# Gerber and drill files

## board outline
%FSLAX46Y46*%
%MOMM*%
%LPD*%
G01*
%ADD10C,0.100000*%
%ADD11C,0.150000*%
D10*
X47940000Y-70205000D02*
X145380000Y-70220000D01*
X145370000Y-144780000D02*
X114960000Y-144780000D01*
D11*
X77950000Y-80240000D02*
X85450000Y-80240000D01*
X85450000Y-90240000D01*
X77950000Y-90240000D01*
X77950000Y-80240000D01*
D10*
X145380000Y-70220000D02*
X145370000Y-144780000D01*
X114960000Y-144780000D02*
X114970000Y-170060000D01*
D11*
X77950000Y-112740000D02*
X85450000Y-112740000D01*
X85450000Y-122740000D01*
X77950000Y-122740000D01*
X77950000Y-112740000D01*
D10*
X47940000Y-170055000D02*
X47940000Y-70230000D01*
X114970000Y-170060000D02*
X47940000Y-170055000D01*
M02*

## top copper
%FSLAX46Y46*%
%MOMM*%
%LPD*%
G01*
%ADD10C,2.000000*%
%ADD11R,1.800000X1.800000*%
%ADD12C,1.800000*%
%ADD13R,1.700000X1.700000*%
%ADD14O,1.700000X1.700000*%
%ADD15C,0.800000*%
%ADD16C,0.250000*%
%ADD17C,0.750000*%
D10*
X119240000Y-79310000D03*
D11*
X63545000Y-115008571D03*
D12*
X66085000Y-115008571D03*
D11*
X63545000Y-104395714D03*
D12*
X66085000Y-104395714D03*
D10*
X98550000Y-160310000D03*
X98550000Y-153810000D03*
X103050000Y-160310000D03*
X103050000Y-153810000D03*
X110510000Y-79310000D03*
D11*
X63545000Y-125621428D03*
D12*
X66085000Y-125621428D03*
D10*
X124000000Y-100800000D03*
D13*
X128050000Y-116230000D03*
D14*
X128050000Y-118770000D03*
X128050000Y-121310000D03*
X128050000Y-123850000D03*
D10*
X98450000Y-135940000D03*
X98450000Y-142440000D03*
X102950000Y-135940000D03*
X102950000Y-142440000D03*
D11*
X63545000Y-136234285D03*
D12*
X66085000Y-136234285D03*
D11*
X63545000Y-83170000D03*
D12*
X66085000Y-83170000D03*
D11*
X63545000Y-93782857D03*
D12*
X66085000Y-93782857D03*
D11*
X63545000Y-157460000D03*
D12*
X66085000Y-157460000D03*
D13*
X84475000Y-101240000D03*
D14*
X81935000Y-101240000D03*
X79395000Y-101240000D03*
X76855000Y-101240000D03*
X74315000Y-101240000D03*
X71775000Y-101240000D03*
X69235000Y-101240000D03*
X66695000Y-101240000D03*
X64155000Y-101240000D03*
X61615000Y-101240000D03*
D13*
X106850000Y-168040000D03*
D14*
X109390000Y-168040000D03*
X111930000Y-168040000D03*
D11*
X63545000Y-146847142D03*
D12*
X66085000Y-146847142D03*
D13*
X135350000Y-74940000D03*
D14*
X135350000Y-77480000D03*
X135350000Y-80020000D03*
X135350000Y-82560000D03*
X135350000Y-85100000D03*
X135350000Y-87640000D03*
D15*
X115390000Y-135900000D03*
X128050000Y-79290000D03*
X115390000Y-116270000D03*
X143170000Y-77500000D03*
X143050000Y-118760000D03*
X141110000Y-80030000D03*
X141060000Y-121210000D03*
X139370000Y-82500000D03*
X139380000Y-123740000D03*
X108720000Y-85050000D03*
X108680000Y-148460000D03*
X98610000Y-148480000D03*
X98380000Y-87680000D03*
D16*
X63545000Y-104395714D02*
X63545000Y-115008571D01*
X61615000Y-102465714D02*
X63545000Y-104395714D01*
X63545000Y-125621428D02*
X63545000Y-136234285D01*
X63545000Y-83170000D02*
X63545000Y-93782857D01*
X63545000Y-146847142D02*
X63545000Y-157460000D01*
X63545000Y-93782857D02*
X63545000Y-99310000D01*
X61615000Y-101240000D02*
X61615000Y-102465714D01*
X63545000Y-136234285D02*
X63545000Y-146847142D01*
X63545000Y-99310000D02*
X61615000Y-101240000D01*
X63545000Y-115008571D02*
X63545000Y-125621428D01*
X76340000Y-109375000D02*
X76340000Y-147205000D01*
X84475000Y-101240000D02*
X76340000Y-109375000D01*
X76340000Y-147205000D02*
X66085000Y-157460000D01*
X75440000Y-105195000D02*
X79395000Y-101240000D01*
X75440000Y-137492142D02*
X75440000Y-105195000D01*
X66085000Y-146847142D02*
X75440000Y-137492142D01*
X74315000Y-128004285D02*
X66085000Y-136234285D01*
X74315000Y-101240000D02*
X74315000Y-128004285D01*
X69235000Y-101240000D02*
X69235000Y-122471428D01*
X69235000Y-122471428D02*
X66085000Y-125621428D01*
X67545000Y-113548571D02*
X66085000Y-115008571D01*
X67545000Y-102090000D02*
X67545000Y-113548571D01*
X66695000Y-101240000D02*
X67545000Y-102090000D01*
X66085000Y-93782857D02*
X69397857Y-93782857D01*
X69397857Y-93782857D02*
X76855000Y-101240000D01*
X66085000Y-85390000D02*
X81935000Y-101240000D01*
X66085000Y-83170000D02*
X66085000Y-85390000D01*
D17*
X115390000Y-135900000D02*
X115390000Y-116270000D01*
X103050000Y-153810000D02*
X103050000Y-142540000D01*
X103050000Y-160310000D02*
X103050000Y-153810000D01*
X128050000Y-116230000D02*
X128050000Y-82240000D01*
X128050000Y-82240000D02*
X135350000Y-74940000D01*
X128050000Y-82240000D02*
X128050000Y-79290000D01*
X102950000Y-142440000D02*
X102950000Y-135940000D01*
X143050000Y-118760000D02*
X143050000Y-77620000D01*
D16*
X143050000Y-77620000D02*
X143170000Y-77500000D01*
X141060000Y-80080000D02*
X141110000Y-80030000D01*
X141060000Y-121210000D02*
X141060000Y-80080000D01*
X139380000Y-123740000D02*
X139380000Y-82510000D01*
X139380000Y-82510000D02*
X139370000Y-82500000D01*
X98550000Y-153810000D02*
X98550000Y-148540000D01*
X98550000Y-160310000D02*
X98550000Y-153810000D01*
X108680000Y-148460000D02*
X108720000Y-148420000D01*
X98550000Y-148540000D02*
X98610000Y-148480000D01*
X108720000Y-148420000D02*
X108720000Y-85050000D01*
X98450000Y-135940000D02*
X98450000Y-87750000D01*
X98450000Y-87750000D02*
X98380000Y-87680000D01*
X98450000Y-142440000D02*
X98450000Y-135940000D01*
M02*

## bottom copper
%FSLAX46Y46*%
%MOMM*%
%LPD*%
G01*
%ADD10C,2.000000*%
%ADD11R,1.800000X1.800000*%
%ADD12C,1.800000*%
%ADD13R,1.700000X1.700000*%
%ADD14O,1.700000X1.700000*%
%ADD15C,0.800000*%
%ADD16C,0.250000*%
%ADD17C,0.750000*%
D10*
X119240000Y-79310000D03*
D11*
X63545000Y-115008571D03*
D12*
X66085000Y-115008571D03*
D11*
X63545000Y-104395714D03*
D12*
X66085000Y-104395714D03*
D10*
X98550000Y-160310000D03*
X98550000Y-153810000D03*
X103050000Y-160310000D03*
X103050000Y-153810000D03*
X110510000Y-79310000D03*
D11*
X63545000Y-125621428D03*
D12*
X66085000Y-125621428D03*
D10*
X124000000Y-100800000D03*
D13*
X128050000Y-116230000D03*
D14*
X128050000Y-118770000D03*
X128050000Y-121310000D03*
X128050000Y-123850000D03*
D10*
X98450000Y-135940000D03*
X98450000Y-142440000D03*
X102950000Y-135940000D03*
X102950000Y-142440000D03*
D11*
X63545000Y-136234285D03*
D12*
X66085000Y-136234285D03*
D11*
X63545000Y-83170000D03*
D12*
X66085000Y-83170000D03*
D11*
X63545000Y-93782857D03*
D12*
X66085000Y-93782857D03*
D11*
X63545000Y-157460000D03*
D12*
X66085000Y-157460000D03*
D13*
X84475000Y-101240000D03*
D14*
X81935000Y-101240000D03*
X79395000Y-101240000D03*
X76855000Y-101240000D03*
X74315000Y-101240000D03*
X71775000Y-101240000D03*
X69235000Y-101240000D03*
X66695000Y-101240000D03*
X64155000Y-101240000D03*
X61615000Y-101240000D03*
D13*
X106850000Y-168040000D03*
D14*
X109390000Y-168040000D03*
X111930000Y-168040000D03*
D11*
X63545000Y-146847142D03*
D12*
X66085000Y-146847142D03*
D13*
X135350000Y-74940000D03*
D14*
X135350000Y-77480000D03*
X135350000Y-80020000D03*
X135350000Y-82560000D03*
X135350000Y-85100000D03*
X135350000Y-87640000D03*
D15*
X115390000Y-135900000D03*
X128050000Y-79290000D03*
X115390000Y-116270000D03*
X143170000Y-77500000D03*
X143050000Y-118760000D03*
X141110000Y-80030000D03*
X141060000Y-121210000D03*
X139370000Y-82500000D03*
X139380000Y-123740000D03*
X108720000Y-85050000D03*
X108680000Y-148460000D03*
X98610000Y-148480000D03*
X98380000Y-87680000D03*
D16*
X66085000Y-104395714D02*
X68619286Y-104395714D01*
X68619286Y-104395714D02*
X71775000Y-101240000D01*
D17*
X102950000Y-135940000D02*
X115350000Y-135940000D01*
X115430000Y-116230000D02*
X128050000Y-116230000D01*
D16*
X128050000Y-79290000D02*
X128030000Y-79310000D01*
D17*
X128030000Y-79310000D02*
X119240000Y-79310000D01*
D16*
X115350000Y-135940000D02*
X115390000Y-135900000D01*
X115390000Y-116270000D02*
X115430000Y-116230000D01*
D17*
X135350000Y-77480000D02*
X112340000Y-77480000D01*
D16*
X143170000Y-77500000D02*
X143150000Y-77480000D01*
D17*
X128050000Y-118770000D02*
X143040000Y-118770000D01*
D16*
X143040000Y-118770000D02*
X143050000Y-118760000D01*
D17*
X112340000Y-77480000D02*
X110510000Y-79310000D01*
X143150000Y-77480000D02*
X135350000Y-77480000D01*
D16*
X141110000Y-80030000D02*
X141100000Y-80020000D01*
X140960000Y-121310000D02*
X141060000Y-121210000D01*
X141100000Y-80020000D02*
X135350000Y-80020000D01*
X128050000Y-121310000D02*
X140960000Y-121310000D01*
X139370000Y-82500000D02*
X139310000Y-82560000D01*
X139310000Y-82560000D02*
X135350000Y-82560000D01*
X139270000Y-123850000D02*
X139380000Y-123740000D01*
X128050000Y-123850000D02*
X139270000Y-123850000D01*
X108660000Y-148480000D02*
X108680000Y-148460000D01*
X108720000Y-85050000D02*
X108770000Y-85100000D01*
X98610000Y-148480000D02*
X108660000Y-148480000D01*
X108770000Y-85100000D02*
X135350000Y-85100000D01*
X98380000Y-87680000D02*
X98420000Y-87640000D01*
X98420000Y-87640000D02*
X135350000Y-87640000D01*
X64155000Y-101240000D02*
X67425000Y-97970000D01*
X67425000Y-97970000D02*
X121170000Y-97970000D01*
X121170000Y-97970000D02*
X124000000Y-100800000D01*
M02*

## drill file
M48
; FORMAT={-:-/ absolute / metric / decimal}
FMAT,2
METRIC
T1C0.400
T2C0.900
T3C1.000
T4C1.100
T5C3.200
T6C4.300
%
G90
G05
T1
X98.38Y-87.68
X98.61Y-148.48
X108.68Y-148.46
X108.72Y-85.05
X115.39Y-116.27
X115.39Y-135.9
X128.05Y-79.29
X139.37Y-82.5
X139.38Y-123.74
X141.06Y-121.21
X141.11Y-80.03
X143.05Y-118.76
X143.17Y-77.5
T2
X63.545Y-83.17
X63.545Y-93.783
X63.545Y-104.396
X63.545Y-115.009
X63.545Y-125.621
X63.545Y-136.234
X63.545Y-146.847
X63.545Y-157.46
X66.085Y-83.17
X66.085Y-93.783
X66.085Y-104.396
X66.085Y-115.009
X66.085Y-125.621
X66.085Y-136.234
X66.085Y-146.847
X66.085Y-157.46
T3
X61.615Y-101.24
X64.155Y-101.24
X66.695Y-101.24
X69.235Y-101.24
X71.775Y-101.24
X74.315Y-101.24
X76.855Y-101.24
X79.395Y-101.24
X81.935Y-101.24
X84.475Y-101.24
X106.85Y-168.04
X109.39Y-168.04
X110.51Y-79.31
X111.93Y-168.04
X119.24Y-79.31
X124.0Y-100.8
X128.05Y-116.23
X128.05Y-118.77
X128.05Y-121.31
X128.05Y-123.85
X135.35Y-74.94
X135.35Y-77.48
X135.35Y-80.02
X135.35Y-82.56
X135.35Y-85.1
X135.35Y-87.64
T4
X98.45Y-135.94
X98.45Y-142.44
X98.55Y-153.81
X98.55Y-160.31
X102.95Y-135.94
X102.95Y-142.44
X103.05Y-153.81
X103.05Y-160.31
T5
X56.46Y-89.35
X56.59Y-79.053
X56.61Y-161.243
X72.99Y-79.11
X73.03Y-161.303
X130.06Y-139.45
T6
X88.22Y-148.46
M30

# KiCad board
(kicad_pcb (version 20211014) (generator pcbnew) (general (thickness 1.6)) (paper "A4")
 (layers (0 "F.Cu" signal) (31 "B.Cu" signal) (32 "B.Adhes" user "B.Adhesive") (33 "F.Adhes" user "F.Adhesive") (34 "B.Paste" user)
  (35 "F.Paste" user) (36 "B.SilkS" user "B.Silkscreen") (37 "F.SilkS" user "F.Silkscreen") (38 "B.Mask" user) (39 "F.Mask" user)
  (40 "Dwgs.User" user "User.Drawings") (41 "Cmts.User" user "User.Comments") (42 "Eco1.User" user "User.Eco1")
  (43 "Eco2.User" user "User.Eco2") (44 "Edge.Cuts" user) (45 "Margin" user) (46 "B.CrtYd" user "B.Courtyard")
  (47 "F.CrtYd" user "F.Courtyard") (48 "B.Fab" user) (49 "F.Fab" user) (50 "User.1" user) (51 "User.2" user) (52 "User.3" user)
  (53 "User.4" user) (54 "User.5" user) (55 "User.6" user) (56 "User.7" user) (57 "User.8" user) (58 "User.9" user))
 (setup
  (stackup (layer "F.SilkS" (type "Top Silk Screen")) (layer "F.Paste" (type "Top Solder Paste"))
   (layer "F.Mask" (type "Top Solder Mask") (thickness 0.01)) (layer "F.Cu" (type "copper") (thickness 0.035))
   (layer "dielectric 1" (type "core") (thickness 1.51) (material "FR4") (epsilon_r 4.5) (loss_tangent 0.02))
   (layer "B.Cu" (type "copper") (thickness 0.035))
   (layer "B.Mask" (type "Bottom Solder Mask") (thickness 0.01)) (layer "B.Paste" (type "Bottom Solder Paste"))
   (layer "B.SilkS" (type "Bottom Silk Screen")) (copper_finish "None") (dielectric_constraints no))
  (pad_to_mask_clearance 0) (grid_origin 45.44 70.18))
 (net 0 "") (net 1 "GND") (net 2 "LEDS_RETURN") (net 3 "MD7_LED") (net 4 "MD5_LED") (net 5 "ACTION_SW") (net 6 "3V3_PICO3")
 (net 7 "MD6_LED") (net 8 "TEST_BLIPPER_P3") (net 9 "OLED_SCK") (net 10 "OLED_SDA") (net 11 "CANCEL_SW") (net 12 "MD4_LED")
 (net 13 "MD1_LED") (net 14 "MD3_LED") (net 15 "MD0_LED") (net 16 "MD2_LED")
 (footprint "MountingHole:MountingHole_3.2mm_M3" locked (layer "F.Cu") (at 130.06 139.450113)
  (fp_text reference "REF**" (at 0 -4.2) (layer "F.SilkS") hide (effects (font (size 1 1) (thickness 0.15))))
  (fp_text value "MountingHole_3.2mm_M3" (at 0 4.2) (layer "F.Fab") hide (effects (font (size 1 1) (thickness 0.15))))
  (pad "" np_thru_hole circle locked (at 0 0) (size 3.2 3.2) (drill 3.2) (layers *.Cu *.Mask)))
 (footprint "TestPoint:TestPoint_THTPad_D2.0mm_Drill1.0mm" (layer "F.Cu") (at 119.24 79.31)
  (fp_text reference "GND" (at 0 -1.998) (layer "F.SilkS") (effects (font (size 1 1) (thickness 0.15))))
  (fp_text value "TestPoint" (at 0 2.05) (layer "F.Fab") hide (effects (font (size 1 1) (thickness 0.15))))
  (pad "1" thru_hole circle (at 0 0) (size 2 2) (drill 1) (layers *.Cu *.Mask) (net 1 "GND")))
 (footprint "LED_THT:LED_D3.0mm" (layer "F.Cu") (at 63.545 115.008571)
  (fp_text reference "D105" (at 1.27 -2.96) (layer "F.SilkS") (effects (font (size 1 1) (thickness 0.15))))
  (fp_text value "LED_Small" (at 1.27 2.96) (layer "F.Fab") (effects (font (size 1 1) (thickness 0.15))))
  (pad "1" thru_hole rect (at 0 0) (size 1.8 1.8) (drill 0.9) (layers *.Cu *.Mask) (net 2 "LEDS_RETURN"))
  (pad "2" thru_hole circle (at 2.54 0) (size 1.8 1.8) (drill 0.9) (layers *.Cu *.Mask) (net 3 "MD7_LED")))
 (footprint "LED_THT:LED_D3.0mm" (layer "F.Cu") (at 63.545 104.395714)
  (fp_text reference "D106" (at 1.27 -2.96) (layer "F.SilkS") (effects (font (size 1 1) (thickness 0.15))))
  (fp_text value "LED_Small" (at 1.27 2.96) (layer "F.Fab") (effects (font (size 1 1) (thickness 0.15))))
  (pad "1" thru_hole rect (at 0 0) (size 1.8 1.8) (drill 0.9) (layers *.Cu *.Mask) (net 2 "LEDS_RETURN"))
  (pad "2" thru_hole circle (at 2.54 0) (size 1.8 1.8) (drill 0.9) (layers *.Cu *.Mask) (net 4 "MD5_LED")))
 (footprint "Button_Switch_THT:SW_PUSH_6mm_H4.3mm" (layer "F.Cu") (at 98.55 160.31 90)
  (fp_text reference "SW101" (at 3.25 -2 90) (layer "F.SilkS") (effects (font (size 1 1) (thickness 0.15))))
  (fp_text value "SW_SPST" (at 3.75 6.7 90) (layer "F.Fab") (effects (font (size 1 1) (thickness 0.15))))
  (pad "1" thru_hole circle (at 0 0 180) (size 2 2) (drill 1.1) (layers *.Cu *.Mask) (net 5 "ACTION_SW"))
  (pad "1" thru_hole circle (at 6.5 0 180) (size 2 2) (drill 1.1) (layers *.Cu *.Mask) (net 5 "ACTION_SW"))
  (pad "2" thru_hole circle (at 0 4.5 180) (size 2 2) (drill 1.1) (layers *.Cu *.Mask) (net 1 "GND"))
  (pad "2" thru_hole circle (at 6.5 4.5 180) (size 2 2) (drill 1.1) (layers *.Cu *.Mask) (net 1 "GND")))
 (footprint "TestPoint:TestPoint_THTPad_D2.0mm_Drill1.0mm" (layer "F.Cu") (at 110.51 79.31)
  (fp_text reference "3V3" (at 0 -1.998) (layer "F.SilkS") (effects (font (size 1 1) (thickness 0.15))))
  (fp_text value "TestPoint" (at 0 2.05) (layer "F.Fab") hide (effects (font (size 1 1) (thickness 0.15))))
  (pad "1" thru_hole circle (at 0 0) (size 2 2) (drill 1) (layers *.Cu *.Mask) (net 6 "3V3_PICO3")))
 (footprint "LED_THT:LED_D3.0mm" (layer "F.Cu") (at 63.545 125.621428)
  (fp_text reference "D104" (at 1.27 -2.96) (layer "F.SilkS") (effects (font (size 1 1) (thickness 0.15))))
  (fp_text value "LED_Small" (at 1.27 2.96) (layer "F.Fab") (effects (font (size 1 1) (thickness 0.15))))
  (pad "1" thru_hole rect (at 0 0) (size 1.8 1.8) (drill 0.9) (layers *.Cu *.Mask) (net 2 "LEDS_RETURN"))
  (pad "2" thru_hole circle (at 2.54 0) (size 1.8 1.8) (drill 0.9) (layers *.Cu *.Mask) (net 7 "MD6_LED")))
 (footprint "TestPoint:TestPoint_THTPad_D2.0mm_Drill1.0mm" (layer "F.Cu") (at 124 100.8)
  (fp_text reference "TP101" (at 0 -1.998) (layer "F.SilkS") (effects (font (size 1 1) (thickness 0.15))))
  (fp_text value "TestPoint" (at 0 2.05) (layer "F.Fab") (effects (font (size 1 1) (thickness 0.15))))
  (pad "1" thru_hole circle (at 0 0) (size 2 2) (drill 1) (layers *.Cu *.Mask) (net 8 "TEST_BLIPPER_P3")))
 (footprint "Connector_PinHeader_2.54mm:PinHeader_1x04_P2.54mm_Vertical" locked (layer "F.Cu") (at 128.05 116.23)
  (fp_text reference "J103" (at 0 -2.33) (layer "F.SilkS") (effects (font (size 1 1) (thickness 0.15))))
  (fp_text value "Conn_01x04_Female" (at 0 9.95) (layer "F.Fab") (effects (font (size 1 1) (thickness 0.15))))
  (pad "1" thru_hole rect locked (at 0 0) (size 1.7 1.7) (drill 1) (layers *.Cu *.Mask) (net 1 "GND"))
  (pad "2" thru_hole oval locked (at 0 2.54) (size 1.7 1.7) (drill 1) (layers *.Cu *.Mask) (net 6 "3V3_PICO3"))
  (pad "3" thru_hole oval locked (at 0 5.08) (size 1.7 1.7) (drill 1) (layers *.Cu *.Mask) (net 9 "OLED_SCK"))
  (pad "4" thru_hole oval locked (at 0 7.62) (size 1.7 1.7) (drill 1) (layers *.Cu *.Mask) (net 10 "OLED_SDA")))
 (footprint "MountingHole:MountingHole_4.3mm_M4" (layer "F.Cu") (at 88.22 148.46)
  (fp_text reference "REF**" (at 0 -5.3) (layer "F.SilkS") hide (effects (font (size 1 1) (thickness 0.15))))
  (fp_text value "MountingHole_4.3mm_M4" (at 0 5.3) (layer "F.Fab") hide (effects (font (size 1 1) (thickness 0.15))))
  (pad "" np_thru_hole circle (at 0 0) (size 4.3 4.3) (drill 4.3) (layers F&B.Cu *.Mask)))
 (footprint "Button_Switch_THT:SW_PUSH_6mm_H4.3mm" (layer "F.Cu") (at 98.45 142.44 90)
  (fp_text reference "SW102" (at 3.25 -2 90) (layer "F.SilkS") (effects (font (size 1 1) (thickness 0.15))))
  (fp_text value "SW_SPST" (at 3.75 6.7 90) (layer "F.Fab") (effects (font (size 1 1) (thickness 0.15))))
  (pad "1" thru_hole circle (at 6.5 0 180) (size 2 2) (drill 1.1) (layers *.Cu *.Mask) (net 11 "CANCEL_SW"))
  (pad "1" thru_hole circle (at 0 0 180) (size 2 2) (drill 1.1) (layers *.Cu *.Mask) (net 11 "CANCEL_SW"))
  (pad "2" thru_hole circle (at 6.5 4.5 180) (size 2 2) (drill 1.1) (layers *.Cu *.Mask) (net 1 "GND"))
  (pad "2" thru_hole circle (at 0 4.5 180) (size 2 2) (drill 1.1) (layers *.Cu *.Mask) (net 1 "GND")))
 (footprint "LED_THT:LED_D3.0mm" (layer "F.Cu") (at 63.545 136.234285)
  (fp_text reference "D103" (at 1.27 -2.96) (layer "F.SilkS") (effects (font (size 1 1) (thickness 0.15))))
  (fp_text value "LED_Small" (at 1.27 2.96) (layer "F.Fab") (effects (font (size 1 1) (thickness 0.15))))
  (pad "1" thru_hole rect (at 0 0) (size 1.8 1.8) (drill 0.9) (layers *.Cu *.Mask) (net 2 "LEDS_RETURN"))
  (pad "2" thru_hole circle (at 2.54 0) (size 1.8 1.8) (drill 0.9) (layers *.Cu *.Mask) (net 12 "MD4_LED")))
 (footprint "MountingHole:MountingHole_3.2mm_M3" (layer "F.Cu") (at 56.59 79.052856 -90)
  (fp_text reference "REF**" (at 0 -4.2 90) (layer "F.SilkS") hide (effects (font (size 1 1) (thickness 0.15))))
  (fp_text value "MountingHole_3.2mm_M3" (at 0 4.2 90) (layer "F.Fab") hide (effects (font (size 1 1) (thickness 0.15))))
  (pad "" np_thru_hole circle locked (at 0 0 270) (size 3.2 3.2) (drill 3.2) (layers F&B.Cu *.Mask)))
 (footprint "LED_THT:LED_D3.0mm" (layer "F.Cu") (at 63.545 83.17)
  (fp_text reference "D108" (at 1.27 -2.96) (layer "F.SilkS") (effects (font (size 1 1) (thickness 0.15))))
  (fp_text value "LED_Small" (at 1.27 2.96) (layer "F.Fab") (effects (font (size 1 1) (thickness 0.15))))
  (pad "1" thru_hole rect (at 0 0) (size 1.8 1.8) (drill 0.9) (layers *.Cu *.Mask) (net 2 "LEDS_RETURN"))
  (pad "2" thru_hole circle (at 2.54 0) (size 1.8 1.8) (drill 0.9) (layers *.Cu *.Mask) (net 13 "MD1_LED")))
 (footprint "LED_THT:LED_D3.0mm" (layer "F.Cu") (at 63.545 93.782857)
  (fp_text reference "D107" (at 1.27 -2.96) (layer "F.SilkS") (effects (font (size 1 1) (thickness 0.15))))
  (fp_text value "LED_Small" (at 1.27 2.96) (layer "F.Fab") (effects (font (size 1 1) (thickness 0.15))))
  (pad "1" thru_hole rect (at 0 0) (size 1.8 1.8) (drill 0.9) (layers *.Cu *.Mask) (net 2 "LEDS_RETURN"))
  (pad "2" thru_hole circle (at 2.54 0) (size 1.8 1.8) (drill 0.9) (layers *.Cu *.Mask) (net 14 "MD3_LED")))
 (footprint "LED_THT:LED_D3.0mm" (layer "F.Cu") (at 63.545 157.46)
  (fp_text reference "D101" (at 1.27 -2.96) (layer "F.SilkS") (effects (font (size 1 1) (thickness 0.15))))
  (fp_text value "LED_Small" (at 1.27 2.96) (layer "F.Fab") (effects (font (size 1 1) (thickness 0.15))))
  (pad "1" thru_hole rect (at 0 0) (size 1.8 1.8) (drill 0.9) (layers *.Cu *.Mask) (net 2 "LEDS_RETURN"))
  (pad "2" thru_hole circle (at 2.54 0) (size 1.8 1.8) (drill 0.9) (layers *.Cu *.Mask) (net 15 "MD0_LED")))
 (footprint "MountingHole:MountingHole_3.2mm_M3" (layer "F.Cu") (at 56.61 161.242856 -90)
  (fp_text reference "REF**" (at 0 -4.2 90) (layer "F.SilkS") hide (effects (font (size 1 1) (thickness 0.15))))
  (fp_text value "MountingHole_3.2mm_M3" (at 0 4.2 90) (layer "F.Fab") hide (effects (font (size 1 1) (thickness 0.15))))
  (pad "" np_thru_hole circle locked (at 0 0 270) (size 3.2 3.2) (drill 3.2) (layers F&B.Cu *.Mask)))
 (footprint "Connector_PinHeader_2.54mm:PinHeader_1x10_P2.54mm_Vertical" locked (layer "F.Cu") (at 84.475 101.24 -90)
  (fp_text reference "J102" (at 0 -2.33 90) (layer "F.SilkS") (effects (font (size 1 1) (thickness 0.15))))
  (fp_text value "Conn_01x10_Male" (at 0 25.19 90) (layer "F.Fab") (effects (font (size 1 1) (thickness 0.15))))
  (pad "1" thru_hole rect locked (at 0 0 270) (size 1.7 1.7) (drill 1) (layers *.Cu *.Mask) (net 15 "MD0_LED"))
  (pad "2" thru_hole oval locked (at 0 2.54 270) (size 1.7 1.7) (drill 1) (layers *.Cu *.Mask) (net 13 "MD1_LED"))
  (pad "3" thru_hole oval locked (at 0 5.08 270) (size 1.7 1.7) (drill 1) (layers *.Cu *.Mask) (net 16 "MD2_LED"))
  (pad "4" thru_hole oval locked (at 0 7.62 270) (size 1.7 1.7) (drill 1) (layers *.Cu *.Mask) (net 14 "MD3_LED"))
  (pad "5" thru_hole oval locked (at 0 10.16 270) (size 1.7 1.7) (drill 1) (layers *.Cu *.Mask) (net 12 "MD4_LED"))
  (pad "6" thru_hole oval locked (at 0 12.7 270) (size 1.7 1.7) (drill 1) (layers *.Cu *.Mask) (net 4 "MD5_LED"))
  (pad "7" thru_hole oval locked (at 0 15.24 270) (size 1.7 1.7) (drill 1) (layers *.Cu *.Mask) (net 7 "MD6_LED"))
  (pad "8" thru_hole oval locked (at 0 17.78 270) (size 1.7 1.7) (drill 1) (layers *.Cu *.Mask) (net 3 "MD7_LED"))
  (pad "9" thru_hole oval locked (at 0 20.32 270) (size 1.7 1.7) (drill 1) (layers *.Cu *.Mask) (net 8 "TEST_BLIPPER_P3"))
  (pad "10" thru_hole oval locked (at 0 22.86 270) (size 1.7 1.7) (drill 1) (layers *.Cu *.Mask) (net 2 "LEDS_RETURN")))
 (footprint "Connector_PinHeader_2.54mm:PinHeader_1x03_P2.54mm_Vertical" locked (layer "F.Cu") (at 106.85 168.04 90)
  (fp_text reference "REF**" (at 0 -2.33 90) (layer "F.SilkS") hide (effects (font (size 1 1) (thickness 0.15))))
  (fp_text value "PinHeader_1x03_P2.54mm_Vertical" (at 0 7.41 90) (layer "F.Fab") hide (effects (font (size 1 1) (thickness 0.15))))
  (pad "1" thru_hole rect locked (at 0 0 90) (size 1.7 1.7) (drill 1) (layers F&B.Cu *.Mask))
  (pad "2" thru_hole oval locked (at 0 2.54 90) (size 1.7 1.7) (drill 1) (layers F&B.Cu *.Mask))
  (pad "3" thru_hole oval locked (at 0 5.08 90) (size 1.7 1.7) (drill 1) (layers F&B.Cu *.Mask)))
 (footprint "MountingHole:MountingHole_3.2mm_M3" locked (layer "F.Cu") (at 56.46 89.350113)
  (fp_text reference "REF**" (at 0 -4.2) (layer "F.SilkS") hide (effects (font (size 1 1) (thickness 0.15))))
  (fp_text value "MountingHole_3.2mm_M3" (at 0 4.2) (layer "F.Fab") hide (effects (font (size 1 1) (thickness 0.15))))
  (pad "" np_thru_hole circle locked (at 0 0) (size 3.2 3.2) (drill 3.2) (layers *.Cu *.Mask)))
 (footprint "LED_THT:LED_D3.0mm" (layer "F.Cu") (at 63.545 146.847142)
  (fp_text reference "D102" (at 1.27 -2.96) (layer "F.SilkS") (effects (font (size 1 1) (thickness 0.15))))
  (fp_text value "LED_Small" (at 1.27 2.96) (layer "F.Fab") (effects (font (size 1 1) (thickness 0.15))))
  (pad "1" thru_hole rect (at 0 0) (size 1.8 1.8) (drill 0.9) (layers *.Cu *.Mask) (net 2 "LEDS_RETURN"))
  (pad "2" thru_hole circle (at 2.54 0) (size 1.8 1.8) (drill 0.9) (layers *.Cu *.Mask) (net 16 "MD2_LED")))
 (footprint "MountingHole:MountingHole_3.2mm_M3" (layer "F.Cu") (at 73.03 161.302856 -90)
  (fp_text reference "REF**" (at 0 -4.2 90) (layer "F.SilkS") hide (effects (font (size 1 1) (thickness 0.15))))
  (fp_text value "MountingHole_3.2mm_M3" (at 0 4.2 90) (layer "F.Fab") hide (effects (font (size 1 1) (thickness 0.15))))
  (pad "" np_thru_hole circle locked (at 0 0 270) (size 3.2 3.2) (drill 3.2) (layers F&B.Cu *.Mask)))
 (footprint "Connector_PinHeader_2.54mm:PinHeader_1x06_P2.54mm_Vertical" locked (layer "F.Cu") (at 135.35 74.94)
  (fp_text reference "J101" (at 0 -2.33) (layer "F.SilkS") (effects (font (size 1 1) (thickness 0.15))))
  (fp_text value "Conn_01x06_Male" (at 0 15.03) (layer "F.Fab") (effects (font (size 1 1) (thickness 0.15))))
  (pad "1" thru_hole rect locked (at 0 0) (size 1.7 1.7) (drill 1) (layers *.Cu *.Mask) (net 1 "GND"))
  (pad "2" thru_hole oval locked (at 0 2.54) (size 1.7 1.7) (drill 1) (layers *.Cu *.Mask) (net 6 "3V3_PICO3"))
  (pad "3" thru_hole oval locked (at 0 5.08) (size 1.7 1.7) (drill 1) (layers *.Cu *.Mask) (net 9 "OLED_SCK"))
  (pad "4" thru_hole oval locked (at 0 7.62) (size 1.7 1.7) (drill 1) (layers *.Cu *.Mask) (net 10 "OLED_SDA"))
  (pad "5" thru_hole oval locked (at 0 10.16) (size 1.7 1.7) (drill 1) (layers *.Cu *.Mask) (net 5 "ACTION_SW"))
  (pad "6" thru_hole oval locked (at 0 12.7) (size 1.7 1.7) (drill 1) (layers *.Cu *.Mask) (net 11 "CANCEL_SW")))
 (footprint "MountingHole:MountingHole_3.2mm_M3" (layer "F.Cu") (at 72.99 79.11)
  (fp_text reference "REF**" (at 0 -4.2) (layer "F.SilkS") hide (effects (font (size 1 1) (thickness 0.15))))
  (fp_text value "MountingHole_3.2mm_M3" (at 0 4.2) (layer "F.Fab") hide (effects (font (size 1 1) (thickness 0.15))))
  (pad "" np_thru_hole circle locked (at 0 0) (size 3.2 3.2) (drill 3.2) (layers F&B.Cu *.Mask)))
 (gr_line (start 47.94 70.205) (end 145.38 70.22) (layer "Edge.Cuts") (width 0.1))
 (gr_line (start 145.37 144.78) (end 114.96 144.78) (layer "Edge.Cuts") (width 0.1))
 (gr_rect (start 77.95 80.24) (end 85.45 90.24) (layer "Edge.Cuts") (width 0.15) (fill none))
 (gr_line (start 145.38 70.22) (end 145.37 144.78) (layer "Edge.Cuts") (width 0.1))
 (gr_line (start 114.96 144.78) (end 114.97 170.06) (layer "Edge.Cuts") (width 0.1))
 (gr_rect (start 77.95 112.74) (end 85.45 122.74) (layer "Edge.Cuts") (width 0.15) (fill none))
 (gr_line (start 47.94 170.055) (end 47.94 70.23) (layer "Edge.Cuts") (width 0.1))
 (gr_line (start 114.97 170.06) (end 47.94 170.055) (layer "Edge.Cuts") (width 0.1))
 (segment (start 63.545 104.395714) (end 63.545 115.008571) (width 0.25) (layer "F.Cu") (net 2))
 (segment (start 61.615 102.465714) (end 63.545 104.395714) (width 0.25) (layer "F.Cu") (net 2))
 (segment (start 63.545 125.621428) (end 63.545 136.234285) (width 0.25) (layer "F.Cu") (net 2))
 (segment (start 63.545 83.17) (end 63.545 93.782857) (width 0.25) (layer "F.Cu") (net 2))
 (segment (start 63.545 146.847142) (end 63.545 157.46) (width 0.25) (layer "F.Cu") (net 2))
 (segment (start 63.545 93.782857) (end 63.545 99.31) (width 0.25) (layer "F.Cu") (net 2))
 (segment (start 61.615 101.24) (end 61.615 102.465714) (width 0.25) (layer "F.Cu") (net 2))
 (segment (start 63.545 136.234285) (end 63.545 146.847142) (width 0.25) (layer "F.Cu") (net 2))
 (segment (start 63.545 99.31) (end 61.615 101.24) (width 0.25) (layer "F.Cu") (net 2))
 (segment (start 63.545 115.008571) (end 63.545 125.621428) (width 0.25) (layer "F.Cu") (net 2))
 (segment (start 76.34 109.375) (end 76.34 147.205) (width 0.25) (layer "F.Cu") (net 15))
 (segment (start 84.475 101.24) (end 76.34 109.375) (width 0.25) (layer "F.Cu") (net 15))
 (segment (start 76.34 147.205) (end 66.085 157.46) (width 0.25) (layer "F.Cu") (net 15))
 (segment (start 75.44 105.195) (end 79.395 101.24) (width 0.25) (layer "F.Cu") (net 16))
 (segment (start 75.44 137.492142) (end 75.44 105.195) (width 0.25) (layer "F.Cu") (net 16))
 (segment (start 66.085 146.847142) (end 75.44 137.492142) (width 0.25) (layer "F.Cu") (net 16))
 (segment (start 74.315 128.004285) (end 66.085 136.234285) (width 0.25) (layer "F.Cu") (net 12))
 (segment (start 74.315 101.24) (end 74.315 128.004285) (width 0.25) (layer "F.Cu") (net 12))
 (segment (start 69.235 101.24) (end 69.235 122.471428) (width 0.25) (layer "F.Cu") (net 7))
 (segment (start 69.235 122.471428) (end 66.085 125.621428) (width 0.25) (layer "F.Cu") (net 7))
 (segment (start 67.545 113.548571) (end 66.085 115.008571) (width 0.25) (layer "F.Cu") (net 3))
 (segment (start 67.545 102.09) (end 67.545 113.548571) (width 0.25) (layer "F.Cu") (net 3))
 (segment (start 66.695 101.24) (end 67.545 102.09) (width 0.25) (layer "F.Cu") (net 3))
 (segment (start 66.085 104.395714) (end 68.619286 104.395714) (width 0.25) (layer "B.Cu") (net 4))
 (segment (start 68.619286 104.395714) (end 71.775 101.24) (width 0.25) (layer "B.Cu") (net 4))
 (segment (start 66.085 93.782857) (end 69.397857 93.782857) (width 0.25) (layer "F.Cu") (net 14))
 (segment (start 69.397857 93.782857) (end 76.855 101.24) (width 0.25) (layer "F.Cu") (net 14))
 (segment (start 66.085 85.39) (end 81.935 101.24) (width 0.25) (layer "F.Cu") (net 13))
 (segment (start 66.085 83.17) (end 66.085 85.39) (width 0.25) (layer "F.Cu") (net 13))
 (segment (start 115.39 135.9) (end 115.39 116.27) (width 0.75) (layer "F.Cu") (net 1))
 (segment (start 103.05 153.81) (end 103.05 142.54) (width 0.75) (layer "F.Cu") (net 1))
 (segment (start 103.05 160.31) (end 103.05 153.81) (width 0.75) (layer "F.Cu") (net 1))
 (segment (start 128.05 116.23) (end 128.05 82.24) (width 0.75) (layer "F.Cu") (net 1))
 (segment (start 128.05 82.24) (end 135.35 74.94) (width 0.75) (layer "F.Cu") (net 1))
 (segment (start 128.05 82.24) (end 128.05 79.29) (width 0.75) (layer "F.Cu") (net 1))
 (segment (start 102.95 142.44) (end 102.95 135.94) (width 0.75) (layer "F.Cu") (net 1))
 (via (at 115.39 135.9) (size 0.8) (drill 0.4) (layers "F.Cu" "B.Cu") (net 1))
 (via (at 128.05 79.29) (size 0.8) (drill 0.4) (layers "F.Cu" "B.Cu") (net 1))
 (via (at 115.39 116.27) (size 0.8) (drill 0.4) (layers "F.Cu" "B.Cu") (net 1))
 (segment (start 102.95 135.94) (end 115.35 135.94) (width 0.75) (layer "B.Cu") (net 1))
 (segment (start 115.43 116.23) (end 128.05 116.23) (width 0.75) (layer "B.Cu") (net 1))
 (segment (start 128.05 79.29) (end 128.03 79.31) (width 0.25) (layer "B.Cu") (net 1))
 (segment (start 128.03 79.31) (end 119.24 79.31) (width 0.75) (layer "B.Cu") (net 1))
 (segment (start 115.35 135.94) (end 115.39 135.9) (width 0.25) (layer "B.Cu") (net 1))
 (segment (start 115.39 116.27) (end 115.43 116.23) (width 0.25) (layer "B.Cu") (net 1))
 (segment (start 143.05 118.76) (end 143.05 77.62) (width 0.75) (layer "F.Cu") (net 6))
 (segment (start 143.05 77.62) (end 143.17 77.5) (width 0.25) (layer "F.Cu") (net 6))
 (via (at 143.17 77.5) (size 0.8) (drill 0.4) (layers "F.Cu" "B.Cu") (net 6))
 (via (at 143.05 118.76) (size 0.8) (drill 0.4) (layers "F.Cu" "B.Cu") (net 6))
 (segment (start 135.35 77.48) (end 112.34 77.48) (width 0.75) (layer "B.Cu") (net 6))
 (segment (start 143.17 77.5) (end 143.15 77.48) (width 0.25) (layer "B.Cu") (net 6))
 (segment (start 128.05 118.77) (end 143.04 118.77) (width 0.75) (layer "B.Cu") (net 6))
 (segment (start 143.04 118.77) (end 143.05 118.76) (width 0.25) (layer "B.Cu") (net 6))
 (segment (start 112.34 77.48) (end 110.51 79.31) (width 0.75) (layer "B.Cu") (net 6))
 (segment (start 143.15 77.48) (end 135.35 77.48) (width 0.75) (layer "B.Cu") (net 6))
 (segment (start 141.06 80.08) (end 141.11 80.03) (width 0.25) (layer "F.Cu") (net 9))
 (segment (start 141.06 121.21) (end 141.06 80.08) (width 0.25) (layer "F.Cu") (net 9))
 (via (at 141.11 80.03) (size 0.8) (drill 0.4) (layers "F.Cu" "B.Cu") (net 9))
 (via (at 141.06 121.21) (size 0.8) (drill 0.4) (layers "F.Cu" "B.Cu") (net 9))
 (segment (start 141.11 80.03) (end 141.1 80.02) (width 0.25) (layer "B.Cu") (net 9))
 (segment (start 140.96 121.31) (end 141.06 121.21) (width 0.25) (layer "B.Cu") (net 9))
 (segment (start 141.1 80.02) (end 135.35 80.02) (width 0.25) (layer "B.Cu") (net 9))
 (segment (start 128.05 121.31) (end 140.96 121.31) (width 0.25) (layer "B.Cu") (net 9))
 (segment (start 139.38 123.74) (end 139.38 82.51) (width 0.25) (layer "F.Cu") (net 10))
 (segment (start 139.38 82.51) (end 139.37 82.5) (width 0.25) (layer "F.Cu") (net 10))
 (via (at 139.37 82.5) (size 0.8) (drill 0.4) (layers "F.Cu" "B.Cu") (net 10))
 (via (at 139.38 123.74) (size 0.8) (drill 0.4) (layers "F.Cu" "B.Cu") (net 10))
 (segment (start 139.37 82.5) (end 139.31 82.56) (width 0.25) (layer "B.Cu") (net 10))
 (segment (start 139.31 82.56) (end 135.35 82.56) (width 0.25) (layer "B.Cu") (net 10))
 (segment (start 139.27 123.85) (end 139.38 123.74) (width 0.25) (layer "B.Cu") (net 10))
 (segment (start 128.05 123.85) (end 139.27 123.85) (width 0.25) (layer "B.Cu") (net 10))
 (segment (start 98.55 153.81) (end 98.55 148.54) (width 0.25) (layer "F.Cu") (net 5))
 (segment (start 98.55 160.31) (end 98.55 153.81) (width 0.25) (layer "F.Cu") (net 5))
 (segment (start 108.68 148.46) (end 108.72 148.42) (width 0.25) (layer "F.Cu") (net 5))
 (segment (start 98.55 148.54) (end 98.61 148.48) (width 0.25) (layer "F.Cu") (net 5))
 (segment (start 108.72 148.42) (end 108.72 85.05) (width 0.25) (layer "F.Cu") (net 5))
 (via (at 108.72 85.05) (size 0.8) (drill 0.4) (layers "F.Cu" "B.Cu") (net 5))
 (via (at 108.68 148.46) (size 0.8) (drill 0.4) (layers "F.Cu" "B.Cu") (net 5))
 (via (at 98.61 148.48) (size 0.8) (drill 0.4) (layers "F.Cu" "B.Cu") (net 5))
 (segment (start 108.66 148.48) (end 108.68 148.46) (width 0.25) (layer "B.Cu") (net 5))
 (segment (start 108.72 85.05) (end 108.77 85.1) (width 0.25) (layer "B.Cu") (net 5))
 (segment (start 98.61 148.48) (end 108.66 148.48) (width 0.25) (layer "B.Cu") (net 5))
 (segment (start 108.77 85.1) (end 135.35 85.1) (width 0.25) (layer "B.Cu") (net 5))
 (segment (start 98.45 135.94) (end 98.45 87.75) (width 0.25) (layer "F.Cu") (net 11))
 (segment (start 98.45 87.75) (end 98.38 87.68) (width 0.25) (layer "F.Cu") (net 11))
 (segment (start 98.45 142.44) (end 98.45 135.94) (width 0.25) (layer "F.Cu") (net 11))
 (via (at 98.38 87.68) (size 0.8) (drill 0.4) (layers "F.Cu" "B.Cu") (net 11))
 (segment (start 98.38 87.68) (end 98.42 87.64) (width 0.25) (layer "B.Cu") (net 11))
 (segment (start 98.42 87.64) (end 135.35 87.64) (width 0.25) (layer "B.Cu") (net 11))
 (segment (start 64.155 101.24) (end 67.425 97.97) (width 0.25) (layer "B.Cu") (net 8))
 (segment (start 67.425 97.97) (end 121.17 97.97) (width 0.25) (layer "B.Cu") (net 8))
 (segment (start 121.17 97.97) (end 124 100.8) (width 0.25) (layer "B.Cu") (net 8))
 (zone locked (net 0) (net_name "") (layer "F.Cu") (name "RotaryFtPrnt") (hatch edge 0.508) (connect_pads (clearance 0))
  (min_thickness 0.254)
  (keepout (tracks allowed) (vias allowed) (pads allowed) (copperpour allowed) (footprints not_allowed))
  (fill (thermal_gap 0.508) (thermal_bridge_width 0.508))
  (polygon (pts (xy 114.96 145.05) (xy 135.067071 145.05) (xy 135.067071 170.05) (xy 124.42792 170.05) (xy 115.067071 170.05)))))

